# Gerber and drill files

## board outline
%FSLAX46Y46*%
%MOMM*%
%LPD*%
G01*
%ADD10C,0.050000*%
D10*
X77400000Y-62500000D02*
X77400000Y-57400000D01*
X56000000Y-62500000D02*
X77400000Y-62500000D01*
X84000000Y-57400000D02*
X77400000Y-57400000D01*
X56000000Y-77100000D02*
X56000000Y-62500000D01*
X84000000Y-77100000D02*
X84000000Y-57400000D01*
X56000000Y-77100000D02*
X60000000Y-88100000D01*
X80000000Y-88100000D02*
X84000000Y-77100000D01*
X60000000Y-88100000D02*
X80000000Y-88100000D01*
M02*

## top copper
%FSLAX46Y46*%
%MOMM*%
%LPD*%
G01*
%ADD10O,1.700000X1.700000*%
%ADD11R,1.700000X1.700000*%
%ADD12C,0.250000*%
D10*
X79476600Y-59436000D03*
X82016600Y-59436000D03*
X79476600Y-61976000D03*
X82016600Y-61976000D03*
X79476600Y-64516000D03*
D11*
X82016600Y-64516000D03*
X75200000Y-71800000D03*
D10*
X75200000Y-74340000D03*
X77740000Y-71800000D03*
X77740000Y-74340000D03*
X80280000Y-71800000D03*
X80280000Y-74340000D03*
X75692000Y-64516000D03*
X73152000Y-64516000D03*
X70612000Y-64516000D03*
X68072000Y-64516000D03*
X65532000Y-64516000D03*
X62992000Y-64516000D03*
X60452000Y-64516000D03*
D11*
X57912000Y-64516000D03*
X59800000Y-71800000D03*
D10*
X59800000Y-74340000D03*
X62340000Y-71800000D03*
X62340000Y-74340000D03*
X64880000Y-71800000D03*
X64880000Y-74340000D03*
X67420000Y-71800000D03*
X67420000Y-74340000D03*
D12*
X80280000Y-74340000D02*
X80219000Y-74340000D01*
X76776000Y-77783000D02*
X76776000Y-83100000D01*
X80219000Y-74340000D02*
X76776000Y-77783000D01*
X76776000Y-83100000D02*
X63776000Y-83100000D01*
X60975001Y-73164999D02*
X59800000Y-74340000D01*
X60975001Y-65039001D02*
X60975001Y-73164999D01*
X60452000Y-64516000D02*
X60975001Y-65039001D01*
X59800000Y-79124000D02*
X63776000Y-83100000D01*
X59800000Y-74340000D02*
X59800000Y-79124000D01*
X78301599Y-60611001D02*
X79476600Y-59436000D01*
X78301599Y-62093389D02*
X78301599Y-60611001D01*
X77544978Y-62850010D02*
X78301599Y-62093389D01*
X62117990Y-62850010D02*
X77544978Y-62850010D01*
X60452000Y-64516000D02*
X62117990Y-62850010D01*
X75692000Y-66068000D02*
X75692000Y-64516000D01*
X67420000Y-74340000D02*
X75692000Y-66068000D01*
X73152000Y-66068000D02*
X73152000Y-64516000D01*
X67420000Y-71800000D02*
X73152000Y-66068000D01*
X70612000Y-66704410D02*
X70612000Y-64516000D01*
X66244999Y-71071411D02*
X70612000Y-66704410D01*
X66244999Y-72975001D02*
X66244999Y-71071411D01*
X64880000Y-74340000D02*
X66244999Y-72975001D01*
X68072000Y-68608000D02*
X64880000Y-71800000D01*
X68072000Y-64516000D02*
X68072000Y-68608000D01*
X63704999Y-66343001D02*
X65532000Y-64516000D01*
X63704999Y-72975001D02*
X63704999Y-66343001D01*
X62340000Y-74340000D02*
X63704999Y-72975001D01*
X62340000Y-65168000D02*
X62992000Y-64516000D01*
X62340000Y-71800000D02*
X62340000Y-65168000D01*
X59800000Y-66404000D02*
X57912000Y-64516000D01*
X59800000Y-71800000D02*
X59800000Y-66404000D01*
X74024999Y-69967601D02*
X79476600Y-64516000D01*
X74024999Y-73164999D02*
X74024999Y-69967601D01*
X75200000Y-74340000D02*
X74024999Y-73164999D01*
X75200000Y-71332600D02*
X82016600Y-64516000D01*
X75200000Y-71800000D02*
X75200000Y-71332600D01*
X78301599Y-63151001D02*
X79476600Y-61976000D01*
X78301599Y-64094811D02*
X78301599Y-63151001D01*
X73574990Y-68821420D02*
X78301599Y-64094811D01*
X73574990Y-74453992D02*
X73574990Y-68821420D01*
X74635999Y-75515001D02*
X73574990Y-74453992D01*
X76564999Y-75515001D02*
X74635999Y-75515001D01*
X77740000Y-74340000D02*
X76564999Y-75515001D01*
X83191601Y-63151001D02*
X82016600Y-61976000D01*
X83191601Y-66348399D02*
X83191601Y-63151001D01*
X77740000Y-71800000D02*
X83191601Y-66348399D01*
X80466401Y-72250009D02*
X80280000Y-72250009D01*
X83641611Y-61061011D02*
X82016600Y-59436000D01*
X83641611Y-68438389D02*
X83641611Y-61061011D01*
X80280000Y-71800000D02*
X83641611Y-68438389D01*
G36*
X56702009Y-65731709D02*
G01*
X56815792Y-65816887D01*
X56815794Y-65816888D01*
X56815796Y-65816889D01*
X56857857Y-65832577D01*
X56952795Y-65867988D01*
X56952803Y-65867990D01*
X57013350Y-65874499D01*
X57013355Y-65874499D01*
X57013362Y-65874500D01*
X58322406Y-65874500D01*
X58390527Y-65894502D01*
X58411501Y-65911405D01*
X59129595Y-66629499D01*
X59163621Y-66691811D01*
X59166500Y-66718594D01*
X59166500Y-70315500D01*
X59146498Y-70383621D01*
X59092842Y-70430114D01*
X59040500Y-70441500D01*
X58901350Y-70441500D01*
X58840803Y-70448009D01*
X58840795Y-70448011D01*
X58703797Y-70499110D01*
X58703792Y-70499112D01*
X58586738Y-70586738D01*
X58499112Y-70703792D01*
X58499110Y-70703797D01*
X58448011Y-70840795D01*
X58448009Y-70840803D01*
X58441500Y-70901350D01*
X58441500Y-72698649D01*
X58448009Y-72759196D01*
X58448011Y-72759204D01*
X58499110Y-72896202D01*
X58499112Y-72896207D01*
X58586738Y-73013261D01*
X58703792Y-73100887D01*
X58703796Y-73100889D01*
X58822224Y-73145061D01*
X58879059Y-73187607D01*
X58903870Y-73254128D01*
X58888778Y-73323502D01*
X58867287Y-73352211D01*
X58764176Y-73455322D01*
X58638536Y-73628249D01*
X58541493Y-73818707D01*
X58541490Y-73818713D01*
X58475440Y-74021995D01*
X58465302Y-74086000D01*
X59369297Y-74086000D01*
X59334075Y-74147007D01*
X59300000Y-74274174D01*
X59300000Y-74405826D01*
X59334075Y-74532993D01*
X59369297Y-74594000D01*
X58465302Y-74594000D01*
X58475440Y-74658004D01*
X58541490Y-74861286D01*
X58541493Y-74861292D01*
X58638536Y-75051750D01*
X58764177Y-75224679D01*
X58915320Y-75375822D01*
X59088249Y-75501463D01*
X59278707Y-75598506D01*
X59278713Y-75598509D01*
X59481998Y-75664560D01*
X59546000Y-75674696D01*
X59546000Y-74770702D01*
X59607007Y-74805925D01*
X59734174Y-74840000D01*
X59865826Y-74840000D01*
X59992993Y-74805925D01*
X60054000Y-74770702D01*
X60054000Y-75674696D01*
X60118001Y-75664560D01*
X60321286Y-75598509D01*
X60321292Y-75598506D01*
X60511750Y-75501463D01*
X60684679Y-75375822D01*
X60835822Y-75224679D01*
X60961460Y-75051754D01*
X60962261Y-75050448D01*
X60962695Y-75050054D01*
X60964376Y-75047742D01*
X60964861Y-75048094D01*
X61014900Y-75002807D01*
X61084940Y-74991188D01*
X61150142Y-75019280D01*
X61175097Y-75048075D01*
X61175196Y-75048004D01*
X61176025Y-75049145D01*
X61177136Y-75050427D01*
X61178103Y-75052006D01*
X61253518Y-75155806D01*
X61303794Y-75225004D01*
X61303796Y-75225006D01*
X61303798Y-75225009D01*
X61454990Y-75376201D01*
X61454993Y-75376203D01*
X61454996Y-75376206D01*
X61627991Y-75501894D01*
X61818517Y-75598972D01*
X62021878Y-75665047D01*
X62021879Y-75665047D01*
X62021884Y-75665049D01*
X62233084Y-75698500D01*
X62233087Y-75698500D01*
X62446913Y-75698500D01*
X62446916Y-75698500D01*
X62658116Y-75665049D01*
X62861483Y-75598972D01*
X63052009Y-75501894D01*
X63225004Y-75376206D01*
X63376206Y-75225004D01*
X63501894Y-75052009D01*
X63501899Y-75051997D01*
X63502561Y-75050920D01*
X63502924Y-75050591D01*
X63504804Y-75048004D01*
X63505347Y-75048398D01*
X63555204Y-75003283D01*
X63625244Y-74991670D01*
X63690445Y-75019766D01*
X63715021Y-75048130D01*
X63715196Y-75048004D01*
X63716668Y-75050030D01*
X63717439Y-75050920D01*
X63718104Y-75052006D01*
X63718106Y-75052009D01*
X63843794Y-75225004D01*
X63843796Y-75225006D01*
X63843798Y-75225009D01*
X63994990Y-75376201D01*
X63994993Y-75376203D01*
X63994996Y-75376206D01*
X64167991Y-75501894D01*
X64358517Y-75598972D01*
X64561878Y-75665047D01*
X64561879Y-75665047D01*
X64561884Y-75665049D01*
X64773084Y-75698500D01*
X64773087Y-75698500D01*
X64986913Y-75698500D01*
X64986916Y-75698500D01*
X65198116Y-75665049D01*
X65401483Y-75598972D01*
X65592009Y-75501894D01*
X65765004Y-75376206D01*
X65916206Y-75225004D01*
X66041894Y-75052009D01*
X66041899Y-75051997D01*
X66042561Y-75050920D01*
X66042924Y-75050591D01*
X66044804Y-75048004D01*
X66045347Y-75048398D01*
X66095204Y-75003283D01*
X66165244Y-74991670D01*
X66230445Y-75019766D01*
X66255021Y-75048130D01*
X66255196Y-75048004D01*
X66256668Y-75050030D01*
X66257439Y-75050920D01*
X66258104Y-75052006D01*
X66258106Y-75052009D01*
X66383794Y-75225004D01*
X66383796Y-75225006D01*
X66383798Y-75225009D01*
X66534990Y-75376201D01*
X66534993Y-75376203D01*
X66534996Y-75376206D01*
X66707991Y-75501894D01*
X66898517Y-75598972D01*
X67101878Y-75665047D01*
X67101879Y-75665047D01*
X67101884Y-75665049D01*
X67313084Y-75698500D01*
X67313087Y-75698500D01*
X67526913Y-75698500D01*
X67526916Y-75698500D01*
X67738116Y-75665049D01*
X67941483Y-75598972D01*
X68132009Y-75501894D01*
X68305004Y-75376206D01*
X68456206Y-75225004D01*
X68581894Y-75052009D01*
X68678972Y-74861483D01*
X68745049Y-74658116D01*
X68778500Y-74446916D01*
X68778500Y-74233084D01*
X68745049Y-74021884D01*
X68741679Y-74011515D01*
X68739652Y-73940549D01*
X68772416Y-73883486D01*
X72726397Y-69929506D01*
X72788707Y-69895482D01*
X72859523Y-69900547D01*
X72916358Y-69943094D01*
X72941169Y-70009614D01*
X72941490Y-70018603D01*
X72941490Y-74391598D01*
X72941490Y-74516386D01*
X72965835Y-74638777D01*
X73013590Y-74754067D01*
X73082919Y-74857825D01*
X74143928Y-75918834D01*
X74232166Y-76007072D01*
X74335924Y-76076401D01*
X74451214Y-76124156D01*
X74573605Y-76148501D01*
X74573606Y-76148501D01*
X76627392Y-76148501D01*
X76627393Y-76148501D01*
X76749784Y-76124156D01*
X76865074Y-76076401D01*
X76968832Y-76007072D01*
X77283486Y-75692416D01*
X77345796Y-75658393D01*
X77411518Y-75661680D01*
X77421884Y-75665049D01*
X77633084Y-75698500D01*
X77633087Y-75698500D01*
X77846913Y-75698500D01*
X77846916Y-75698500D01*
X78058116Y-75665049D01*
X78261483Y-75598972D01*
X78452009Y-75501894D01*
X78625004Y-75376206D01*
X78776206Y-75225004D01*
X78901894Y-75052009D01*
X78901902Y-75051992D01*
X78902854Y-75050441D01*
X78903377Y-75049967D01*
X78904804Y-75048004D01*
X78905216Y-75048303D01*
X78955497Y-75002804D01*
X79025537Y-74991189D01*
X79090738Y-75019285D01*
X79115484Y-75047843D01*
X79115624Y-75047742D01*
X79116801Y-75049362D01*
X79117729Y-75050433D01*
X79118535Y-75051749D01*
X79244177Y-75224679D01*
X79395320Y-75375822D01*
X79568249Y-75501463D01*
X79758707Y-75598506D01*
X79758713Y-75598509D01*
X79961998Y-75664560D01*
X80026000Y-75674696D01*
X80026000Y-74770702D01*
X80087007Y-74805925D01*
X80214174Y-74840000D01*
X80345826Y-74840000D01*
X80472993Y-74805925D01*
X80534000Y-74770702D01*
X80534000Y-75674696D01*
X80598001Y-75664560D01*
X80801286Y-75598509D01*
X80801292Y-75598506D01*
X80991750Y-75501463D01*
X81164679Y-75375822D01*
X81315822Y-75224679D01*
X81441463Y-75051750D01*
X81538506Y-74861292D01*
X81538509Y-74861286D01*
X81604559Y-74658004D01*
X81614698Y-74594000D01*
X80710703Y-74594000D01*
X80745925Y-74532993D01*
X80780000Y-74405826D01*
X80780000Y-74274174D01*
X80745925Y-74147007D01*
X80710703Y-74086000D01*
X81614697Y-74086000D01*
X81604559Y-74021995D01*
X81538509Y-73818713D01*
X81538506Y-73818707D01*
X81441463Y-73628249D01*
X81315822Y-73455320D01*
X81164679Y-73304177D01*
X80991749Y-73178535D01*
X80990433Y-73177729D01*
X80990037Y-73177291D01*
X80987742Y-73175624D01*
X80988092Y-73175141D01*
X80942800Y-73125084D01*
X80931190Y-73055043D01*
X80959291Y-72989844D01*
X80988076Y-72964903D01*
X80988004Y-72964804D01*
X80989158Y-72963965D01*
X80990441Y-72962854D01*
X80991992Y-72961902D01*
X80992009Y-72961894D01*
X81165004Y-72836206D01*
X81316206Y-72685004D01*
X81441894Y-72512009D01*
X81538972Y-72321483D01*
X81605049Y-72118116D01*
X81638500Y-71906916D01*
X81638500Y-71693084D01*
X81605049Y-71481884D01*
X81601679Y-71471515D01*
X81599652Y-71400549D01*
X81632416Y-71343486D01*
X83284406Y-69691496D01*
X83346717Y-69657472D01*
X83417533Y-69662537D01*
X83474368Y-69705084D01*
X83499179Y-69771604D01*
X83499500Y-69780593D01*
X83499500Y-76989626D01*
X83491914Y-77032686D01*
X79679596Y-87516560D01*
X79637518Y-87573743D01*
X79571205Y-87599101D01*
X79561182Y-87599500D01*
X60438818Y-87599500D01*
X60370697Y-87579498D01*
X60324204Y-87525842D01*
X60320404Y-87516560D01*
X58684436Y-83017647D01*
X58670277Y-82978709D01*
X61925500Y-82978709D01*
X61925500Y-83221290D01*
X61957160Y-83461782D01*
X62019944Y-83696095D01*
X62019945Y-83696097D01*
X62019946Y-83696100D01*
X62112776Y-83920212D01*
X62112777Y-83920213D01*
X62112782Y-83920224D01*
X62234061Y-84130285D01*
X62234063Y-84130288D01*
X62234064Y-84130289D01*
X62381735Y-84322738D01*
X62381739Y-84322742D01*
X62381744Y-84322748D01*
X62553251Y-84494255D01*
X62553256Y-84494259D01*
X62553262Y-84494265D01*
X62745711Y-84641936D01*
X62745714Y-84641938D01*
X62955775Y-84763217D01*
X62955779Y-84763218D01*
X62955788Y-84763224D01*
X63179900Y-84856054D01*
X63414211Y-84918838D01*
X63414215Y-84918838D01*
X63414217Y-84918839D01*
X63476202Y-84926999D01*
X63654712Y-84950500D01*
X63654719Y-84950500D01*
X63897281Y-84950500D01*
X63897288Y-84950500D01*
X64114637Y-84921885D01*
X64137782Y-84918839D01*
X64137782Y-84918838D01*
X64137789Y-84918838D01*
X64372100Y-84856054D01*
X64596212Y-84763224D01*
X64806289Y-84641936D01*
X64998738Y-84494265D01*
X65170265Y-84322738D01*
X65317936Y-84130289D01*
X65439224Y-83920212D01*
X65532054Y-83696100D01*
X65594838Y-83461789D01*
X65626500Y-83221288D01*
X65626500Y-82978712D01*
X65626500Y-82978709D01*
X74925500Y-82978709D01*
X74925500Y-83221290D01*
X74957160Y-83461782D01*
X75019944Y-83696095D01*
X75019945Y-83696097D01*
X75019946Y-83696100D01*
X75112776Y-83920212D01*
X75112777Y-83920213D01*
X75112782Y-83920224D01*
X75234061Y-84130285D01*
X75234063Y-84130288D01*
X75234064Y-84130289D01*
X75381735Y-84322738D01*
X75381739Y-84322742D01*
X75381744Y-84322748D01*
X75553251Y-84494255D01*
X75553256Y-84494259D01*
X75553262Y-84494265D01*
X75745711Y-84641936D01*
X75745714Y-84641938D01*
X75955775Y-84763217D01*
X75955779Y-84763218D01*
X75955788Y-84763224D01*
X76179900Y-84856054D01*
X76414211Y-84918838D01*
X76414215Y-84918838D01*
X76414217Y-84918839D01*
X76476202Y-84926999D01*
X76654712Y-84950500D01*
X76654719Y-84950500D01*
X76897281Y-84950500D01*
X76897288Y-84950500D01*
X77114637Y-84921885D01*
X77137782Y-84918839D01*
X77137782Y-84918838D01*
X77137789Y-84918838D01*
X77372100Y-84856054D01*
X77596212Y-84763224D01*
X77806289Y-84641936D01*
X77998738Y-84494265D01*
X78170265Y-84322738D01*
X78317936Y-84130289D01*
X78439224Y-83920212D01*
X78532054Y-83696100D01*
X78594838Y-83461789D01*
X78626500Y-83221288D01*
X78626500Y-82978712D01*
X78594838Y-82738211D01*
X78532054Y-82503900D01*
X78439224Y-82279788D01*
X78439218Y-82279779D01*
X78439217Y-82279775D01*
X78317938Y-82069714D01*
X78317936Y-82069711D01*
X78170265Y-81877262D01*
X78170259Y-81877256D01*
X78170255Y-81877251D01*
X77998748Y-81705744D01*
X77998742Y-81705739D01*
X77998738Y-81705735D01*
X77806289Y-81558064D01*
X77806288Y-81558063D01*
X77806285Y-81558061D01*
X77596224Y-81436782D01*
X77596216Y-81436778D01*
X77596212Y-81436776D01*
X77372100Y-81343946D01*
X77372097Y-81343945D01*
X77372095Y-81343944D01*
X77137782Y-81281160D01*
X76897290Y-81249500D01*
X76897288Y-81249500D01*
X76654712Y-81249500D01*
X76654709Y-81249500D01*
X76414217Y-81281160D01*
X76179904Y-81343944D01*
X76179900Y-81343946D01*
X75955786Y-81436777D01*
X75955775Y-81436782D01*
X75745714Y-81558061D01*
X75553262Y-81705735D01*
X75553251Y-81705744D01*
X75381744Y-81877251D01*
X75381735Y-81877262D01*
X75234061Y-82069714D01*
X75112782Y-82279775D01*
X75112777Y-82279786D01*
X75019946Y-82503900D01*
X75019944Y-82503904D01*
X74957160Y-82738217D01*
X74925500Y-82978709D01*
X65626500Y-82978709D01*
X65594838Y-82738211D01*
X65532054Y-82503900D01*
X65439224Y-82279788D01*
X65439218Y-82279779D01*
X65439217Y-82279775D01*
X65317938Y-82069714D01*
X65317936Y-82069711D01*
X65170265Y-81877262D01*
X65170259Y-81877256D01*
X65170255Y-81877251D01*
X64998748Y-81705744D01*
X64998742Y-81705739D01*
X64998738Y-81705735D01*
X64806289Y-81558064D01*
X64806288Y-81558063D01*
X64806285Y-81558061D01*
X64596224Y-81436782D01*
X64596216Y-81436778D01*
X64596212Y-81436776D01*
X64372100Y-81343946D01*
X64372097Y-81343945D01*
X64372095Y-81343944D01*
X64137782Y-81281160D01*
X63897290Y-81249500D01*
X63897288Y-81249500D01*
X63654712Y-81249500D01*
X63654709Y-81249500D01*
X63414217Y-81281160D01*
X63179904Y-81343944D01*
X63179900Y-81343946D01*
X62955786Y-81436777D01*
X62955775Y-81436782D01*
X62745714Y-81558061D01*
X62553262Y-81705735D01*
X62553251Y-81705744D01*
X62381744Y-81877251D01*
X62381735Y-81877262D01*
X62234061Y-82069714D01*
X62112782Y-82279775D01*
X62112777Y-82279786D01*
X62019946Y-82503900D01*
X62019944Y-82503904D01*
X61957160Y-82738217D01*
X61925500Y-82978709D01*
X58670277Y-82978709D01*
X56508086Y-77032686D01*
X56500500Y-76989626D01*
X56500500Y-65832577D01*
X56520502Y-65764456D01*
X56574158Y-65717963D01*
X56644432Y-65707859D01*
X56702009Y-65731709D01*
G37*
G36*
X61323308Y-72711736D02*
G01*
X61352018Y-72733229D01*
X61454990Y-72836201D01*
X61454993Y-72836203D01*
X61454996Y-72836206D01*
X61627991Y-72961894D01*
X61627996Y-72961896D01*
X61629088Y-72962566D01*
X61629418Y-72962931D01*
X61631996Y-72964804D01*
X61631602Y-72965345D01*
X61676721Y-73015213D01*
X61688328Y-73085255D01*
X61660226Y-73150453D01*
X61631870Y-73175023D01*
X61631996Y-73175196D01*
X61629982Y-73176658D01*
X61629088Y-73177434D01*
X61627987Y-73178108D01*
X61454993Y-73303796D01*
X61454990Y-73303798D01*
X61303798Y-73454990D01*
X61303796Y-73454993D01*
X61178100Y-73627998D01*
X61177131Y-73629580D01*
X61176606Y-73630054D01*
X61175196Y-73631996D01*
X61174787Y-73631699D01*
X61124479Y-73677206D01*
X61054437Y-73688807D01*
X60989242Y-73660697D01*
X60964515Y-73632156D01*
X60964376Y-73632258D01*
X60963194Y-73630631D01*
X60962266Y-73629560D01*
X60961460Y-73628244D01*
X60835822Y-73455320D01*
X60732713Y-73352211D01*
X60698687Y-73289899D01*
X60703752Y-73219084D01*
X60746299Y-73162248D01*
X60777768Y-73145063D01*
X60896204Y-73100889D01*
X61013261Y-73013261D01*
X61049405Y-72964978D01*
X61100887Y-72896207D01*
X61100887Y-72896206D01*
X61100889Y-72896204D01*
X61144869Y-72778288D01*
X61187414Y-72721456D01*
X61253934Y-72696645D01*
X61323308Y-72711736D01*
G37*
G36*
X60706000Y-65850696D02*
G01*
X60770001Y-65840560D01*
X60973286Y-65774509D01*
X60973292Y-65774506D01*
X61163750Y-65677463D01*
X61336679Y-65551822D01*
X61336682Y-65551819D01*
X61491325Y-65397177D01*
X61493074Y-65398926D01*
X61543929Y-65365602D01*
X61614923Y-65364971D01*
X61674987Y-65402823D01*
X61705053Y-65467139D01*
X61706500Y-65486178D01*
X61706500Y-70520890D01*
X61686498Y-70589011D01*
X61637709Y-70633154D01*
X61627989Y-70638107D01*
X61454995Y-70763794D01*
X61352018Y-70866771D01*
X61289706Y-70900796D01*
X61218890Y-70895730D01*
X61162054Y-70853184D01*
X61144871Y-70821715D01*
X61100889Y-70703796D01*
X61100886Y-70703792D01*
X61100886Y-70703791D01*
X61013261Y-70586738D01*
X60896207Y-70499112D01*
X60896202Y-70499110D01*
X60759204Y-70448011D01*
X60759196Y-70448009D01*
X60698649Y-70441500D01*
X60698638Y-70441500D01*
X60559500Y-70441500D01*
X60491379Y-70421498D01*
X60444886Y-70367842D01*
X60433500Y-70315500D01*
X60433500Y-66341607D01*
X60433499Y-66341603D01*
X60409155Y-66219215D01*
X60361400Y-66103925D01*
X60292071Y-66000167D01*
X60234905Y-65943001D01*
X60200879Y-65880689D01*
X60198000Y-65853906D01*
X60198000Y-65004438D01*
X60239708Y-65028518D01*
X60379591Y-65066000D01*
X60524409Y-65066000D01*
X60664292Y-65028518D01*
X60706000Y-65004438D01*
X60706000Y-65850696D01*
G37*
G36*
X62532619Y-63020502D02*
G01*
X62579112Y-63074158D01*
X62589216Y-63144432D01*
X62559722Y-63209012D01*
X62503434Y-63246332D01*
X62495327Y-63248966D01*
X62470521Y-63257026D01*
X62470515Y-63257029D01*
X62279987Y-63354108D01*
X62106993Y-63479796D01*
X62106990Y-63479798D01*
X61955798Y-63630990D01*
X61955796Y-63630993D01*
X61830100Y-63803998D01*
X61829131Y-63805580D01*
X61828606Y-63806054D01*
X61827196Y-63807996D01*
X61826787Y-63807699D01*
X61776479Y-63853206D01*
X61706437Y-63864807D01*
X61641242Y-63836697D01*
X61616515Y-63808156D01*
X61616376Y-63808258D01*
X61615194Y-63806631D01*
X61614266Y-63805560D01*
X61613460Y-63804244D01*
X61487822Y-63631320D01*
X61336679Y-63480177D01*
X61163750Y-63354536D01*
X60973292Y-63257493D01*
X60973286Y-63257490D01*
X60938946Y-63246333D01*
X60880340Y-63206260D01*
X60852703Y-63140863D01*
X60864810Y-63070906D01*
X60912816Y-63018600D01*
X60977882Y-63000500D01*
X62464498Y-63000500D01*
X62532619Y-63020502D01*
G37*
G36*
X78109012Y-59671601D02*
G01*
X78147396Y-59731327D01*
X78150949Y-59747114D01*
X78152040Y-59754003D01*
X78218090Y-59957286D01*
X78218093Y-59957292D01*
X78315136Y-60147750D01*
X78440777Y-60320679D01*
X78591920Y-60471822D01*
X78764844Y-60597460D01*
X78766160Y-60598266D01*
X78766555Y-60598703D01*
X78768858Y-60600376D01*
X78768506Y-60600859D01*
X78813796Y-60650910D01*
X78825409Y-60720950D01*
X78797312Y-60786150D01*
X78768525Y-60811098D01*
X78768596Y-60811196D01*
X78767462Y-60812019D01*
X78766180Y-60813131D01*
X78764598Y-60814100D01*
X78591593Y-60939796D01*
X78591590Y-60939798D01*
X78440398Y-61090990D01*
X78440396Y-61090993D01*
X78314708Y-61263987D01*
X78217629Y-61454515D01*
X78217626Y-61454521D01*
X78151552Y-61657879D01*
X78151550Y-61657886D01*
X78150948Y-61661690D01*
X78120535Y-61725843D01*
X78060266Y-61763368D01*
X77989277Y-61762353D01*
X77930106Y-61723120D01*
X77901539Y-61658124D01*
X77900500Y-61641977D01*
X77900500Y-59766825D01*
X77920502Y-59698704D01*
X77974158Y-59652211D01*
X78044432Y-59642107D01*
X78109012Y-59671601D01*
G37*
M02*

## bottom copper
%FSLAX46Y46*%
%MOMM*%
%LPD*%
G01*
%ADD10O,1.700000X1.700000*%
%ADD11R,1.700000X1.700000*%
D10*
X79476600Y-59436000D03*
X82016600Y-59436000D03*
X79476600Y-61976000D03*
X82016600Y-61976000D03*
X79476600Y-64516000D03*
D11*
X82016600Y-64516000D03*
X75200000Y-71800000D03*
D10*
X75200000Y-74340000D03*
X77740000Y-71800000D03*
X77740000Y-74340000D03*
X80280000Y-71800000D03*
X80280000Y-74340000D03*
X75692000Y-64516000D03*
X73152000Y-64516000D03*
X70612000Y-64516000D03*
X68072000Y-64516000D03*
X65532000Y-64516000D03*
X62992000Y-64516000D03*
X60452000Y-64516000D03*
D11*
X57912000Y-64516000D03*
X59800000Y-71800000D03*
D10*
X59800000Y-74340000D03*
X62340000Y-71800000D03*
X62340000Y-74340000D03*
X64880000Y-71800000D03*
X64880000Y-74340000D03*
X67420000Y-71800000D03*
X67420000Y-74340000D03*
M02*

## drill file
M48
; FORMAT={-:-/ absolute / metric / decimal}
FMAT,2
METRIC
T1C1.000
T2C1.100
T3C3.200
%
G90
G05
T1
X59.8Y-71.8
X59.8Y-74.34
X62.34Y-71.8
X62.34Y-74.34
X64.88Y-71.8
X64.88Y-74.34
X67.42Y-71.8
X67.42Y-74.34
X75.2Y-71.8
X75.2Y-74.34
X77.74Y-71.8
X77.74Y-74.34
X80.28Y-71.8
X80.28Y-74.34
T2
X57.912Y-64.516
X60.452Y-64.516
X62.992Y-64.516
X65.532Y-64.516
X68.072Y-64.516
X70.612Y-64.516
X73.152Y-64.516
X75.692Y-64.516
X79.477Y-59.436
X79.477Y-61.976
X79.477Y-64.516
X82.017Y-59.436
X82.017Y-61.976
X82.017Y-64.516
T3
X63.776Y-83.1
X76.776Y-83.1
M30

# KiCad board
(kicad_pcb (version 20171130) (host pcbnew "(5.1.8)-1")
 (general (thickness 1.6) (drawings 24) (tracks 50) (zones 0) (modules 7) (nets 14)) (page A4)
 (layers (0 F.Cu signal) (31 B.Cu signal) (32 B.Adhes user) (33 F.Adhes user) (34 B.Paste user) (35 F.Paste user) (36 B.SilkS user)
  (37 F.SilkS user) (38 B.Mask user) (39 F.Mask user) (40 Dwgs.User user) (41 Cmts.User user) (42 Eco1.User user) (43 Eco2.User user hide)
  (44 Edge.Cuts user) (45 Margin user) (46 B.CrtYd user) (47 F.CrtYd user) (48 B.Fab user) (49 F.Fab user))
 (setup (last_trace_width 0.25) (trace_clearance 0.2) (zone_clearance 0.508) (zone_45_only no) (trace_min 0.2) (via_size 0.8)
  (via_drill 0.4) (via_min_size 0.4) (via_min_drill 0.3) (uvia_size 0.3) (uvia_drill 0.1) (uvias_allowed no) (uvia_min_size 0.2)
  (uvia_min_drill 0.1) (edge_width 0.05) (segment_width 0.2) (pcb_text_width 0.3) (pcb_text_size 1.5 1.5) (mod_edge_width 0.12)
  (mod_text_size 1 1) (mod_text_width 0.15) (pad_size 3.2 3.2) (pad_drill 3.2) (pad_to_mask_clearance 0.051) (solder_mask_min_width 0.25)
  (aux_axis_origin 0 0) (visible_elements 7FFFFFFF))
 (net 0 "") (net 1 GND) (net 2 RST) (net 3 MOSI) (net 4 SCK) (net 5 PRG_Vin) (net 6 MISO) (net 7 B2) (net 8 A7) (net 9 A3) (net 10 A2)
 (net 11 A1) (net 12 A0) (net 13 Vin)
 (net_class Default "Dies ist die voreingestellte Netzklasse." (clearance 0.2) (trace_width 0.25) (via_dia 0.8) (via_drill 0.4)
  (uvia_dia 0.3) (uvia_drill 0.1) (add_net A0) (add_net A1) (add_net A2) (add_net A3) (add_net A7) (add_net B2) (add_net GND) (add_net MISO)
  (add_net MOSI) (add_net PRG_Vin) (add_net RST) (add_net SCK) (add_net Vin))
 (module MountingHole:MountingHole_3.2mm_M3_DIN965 (layer F.Cu) (at 63.6778 83.1342)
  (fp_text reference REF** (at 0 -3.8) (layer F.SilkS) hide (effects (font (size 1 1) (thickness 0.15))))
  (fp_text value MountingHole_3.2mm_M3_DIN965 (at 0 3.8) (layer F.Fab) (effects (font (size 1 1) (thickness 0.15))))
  (pad "" np_thru_hole circle (at 0.0982 -0.0342) (size 3.2 3.2) (drill 3.2) (layers *.Cu *.Mask)))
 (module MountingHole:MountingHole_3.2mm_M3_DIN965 (layer F.Cu) (at 76.776 83.1)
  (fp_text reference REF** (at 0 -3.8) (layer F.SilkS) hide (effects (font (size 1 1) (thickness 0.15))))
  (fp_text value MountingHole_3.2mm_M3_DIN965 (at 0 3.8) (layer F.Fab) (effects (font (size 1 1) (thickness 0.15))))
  (pad 1 np_thru_hole circle (at 0 0) (size 3.2 3.2) (drill 3.2) (layers *.Cu *.Mask)))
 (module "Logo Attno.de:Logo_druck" (layer F.Cu) (at 70.2056 82.042)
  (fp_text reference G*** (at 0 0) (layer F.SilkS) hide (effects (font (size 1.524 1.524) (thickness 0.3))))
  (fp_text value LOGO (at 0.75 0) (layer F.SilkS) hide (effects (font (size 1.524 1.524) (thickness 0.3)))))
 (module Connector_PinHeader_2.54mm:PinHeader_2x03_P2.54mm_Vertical (layer F.Cu) (at 82.0166 64.516 180)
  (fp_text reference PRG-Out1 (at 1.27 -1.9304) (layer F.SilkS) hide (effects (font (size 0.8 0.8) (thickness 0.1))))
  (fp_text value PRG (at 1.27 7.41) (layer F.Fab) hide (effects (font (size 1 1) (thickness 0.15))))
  (pad 6 thru_hole oval (at 2.54 5.08 180) (size 1.7 1.7) (drill 1.1) (layers *.Cu *.Mask) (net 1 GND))
  (pad 5 thru_hole oval (at 0 5.08 180) (size 1.7 1.7) (drill 1.1) (layers *.Cu *.Mask) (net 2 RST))
  (pad 4 thru_hole oval (at 2.54 2.54 180) (size 1.7 1.7) (drill 1.1) (layers *.Cu *.Mask) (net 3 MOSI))
  (pad 3 thru_hole oval (at 0 2.54 180) (size 1.7 1.7) (drill 1.1) (layers *.Cu *.Mask) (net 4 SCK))
  (pad 2 thru_hole oval (at 2.54 0 180) (size 1.7 1.7) (drill 1.1) (layers *.Cu *.Mask) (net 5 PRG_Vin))
  (pad 1 thru_hole rect (at 0 0 180) (size 1.7 1.7) (drill 1.1) (layers *.Cu *.Mask) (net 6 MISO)))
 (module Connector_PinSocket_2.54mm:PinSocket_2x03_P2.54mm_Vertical (layer F.Cu) (at 75.2 71.8 90)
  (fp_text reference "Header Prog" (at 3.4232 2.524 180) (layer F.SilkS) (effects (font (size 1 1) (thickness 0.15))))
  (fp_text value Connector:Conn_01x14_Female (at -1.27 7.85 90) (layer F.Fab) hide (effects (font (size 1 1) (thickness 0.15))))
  (pad 1 thru_hole rect (at 0 0 90) (size 1.7 1.7) (drill 1) (layers *.Cu *.Mask) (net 6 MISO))
  (pad 2 thru_hole oval (at -2.54 0 90) (size 1.7 1.7) (drill 1) (layers *.Cu *.Mask) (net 5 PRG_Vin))
  (pad 3 thru_hole oval (at 0 2.54 90) (size 1.7 1.7) (drill 1) (layers *.Cu *.Mask) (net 4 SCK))
  (pad 4 thru_hole oval (at -2.54 2.54 90) (size 1.7 1.7) (drill 1) (layers *.Cu *.Mask) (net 3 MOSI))
  (pad 5 thru_hole oval (at 0 5.08 90) (size 1.7 1.7) (drill 1) (layers *.Cu *.Mask) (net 2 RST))
  (pad 6 thru_hole oval (at -2.54 5.08 90) (size 1.7 1.7) (drill 1) (layers *.Cu *.Mask) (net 1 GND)))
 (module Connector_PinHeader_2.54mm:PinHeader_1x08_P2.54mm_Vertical (layer F.Cu) (at 57.912 64.516 90)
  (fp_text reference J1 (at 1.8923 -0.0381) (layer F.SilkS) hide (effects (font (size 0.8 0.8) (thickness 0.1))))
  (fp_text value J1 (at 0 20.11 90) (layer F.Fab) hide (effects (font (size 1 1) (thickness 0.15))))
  (pad 8 thru_hole oval (at 0 17.78 90) (size 1.7 1.7) (drill 1.1) (layers *.Cu *.Mask) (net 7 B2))
  (pad 7 thru_hole oval (at 0 15.24 90) (size 1.7 1.7) (drill 1.1) (layers *.Cu *.Mask) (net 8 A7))
  (pad 6 thru_hole oval (at 0 12.7 90) (size 1.7 1.7) (drill 1.1) (layers *.Cu *.Mask) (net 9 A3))
  (pad 5 thru_hole oval (at 0 10.16 90) (size 1.7 1.7) (drill 1.1) (layers *.Cu *.Mask) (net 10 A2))
  (pad 4 thru_hole oval (at 0 7.62 90) (size 1.7 1.7) (drill 1.1) (layers *.Cu *.Mask) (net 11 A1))
  (pad 3 thru_hole oval (at 0 5.08 90) (size 1.7 1.7) (drill 1.1) (layers *.Cu *.Mask) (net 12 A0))
  (pad 2 thru_hole oval (at 0 2.54 90) (size 1.7 1.7) (drill 1.1) (layers *.Cu *.Mask) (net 1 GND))
  (pad 1 thru_hole rect (at 0 0 90) (size 1.7 1.7) (drill 1.1) (layers *.Cu *.Mask) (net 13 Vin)))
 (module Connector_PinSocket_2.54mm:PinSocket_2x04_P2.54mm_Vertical (layer F.Cu) (at 59.8 71.8 90)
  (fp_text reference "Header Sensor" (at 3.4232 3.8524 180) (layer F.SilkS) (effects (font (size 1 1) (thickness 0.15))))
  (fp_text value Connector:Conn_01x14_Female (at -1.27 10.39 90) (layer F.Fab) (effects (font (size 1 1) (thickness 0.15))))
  (pad 1 thru_hole rect (at 0 0 90) (size 1.7 1.7) (drill 1) (layers *.Cu *.Mask) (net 13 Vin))
  (pad 2 thru_hole oval (at -2.54 0 90) (size 1.7 1.7) (drill 1) (layers *.Cu *.Mask) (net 1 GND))
  (pad 3 thru_hole oval (at 0 2.54 90) (size 1.7 1.7) (drill 1) (layers *.Cu *.Mask) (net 12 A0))
  (pad 4 thru_hole oval (at -2.54 2.54 90) (size 1.7 1.7) (drill 1) (layers *.Cu *.Mask) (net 11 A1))
  (pad 5 thru_hole oval (at 0 5.08 90) (size 1.7 1.7) (drill 1) (layers *.Cu *.Mask) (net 10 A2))
  (pad 6 thru_hole oval (at -2.54 5.08 90) (size 1.7 1.7) (drill 1) (layers *.Cu *.Mask) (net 9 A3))
  (pad 7 thru_hole oval (at 0 7.62 90) (size 1.7 1.7) (drill 1) (layers *.Cu *.Mask) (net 8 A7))
  (pad 8 thru_hole oval (at -2.54 7.62 90) (size 1.7 1.7) (drill 1) (layers *.Cu *.Mask) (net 7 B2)))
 (gr_line (start 77.4 62.5) (end 77.4 57.4) (layer Edge.Cuts) (width 0.05))
 (gr_line (start 56 62.5) (end 77.4 62.5) (layer Edge.Cuts) (width 0.05))
 (gr_line (start 84 57.4) (end 77.4 57.4) (layer Edge.Cuts) (width 0.05))
 (gr_line (start 56 77.1) (end 56 62.5) (layer Edge.Cuts) (width 0.05))
 (gr_line (start 84 77.1) (end 84 57.4) (layer Edge.Cuts) (width 0.05))
 (gr_line (start 56 77.1) (end 60 88.1) (layer Edge.Cuts) (width 0.05))
 (gr_line (start 80 88.1) (end 84 77.1) (layer Edge.Cuts) (width 0.05))
 (gr_line (start 60 88.1) (end 80 88.1) (layer Edge.Cuts) (width 0.05))
 (segment (start 80.28 74.34) (end 80.219 74.34) (width 0.25) (layer F.Cu) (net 1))
 (segment (start 76.776 77.783) (end 76.776 83.1) (width 0.25) (layer F.Cu) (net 1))
 (segment (start 80.219 74.34) (end 76.776 77.783) (width 0.25) (layer F.Cu) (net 1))
 (segment (start 76.776 83.1) (end 63.776 83.1) (width 0.25) (layer F.Cu) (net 1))
 (segment (start 60.975001 73.164999) (end 59.8 74.34) (width 0.25) (layer F.Cu) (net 1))
 (segment (start 60.975001 65.039001) (end 60.975001 73.164999) (width 0.25) (layer F.Cu) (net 1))
 (segment (start 60.452 64.516) (end 60.975001 65.039001) (width 0.25) (layer F.Cu) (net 1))
 (segment (start 59.8 79.124) (end 63.776 83.1) (width 0.25) (layer F.Cu) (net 1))
 (segment (start 59.8 74.34) (end 59.8 79.124) (width 0.25) (layer F.Cu) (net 1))
 (segment (start 78.301599 60.611001) (end 79.4766 59.436) (width 0.25) (layer F.Cu) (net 1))
 (segment (start 78.301599 62.093389) (end 78.301599 60.611001) (width 0.25) (layer F.Cu) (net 1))
 (segment (start 77.544978 62.85001) (end 78.301599 62.093389) (width 0.25) (layer F.Cu) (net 1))
 (segment (start 62.11799 62.85001) (end 77.544978 62.85001) (width 0.25) (layer F.Cu) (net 1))
 (segment (start 60.452 64.516) (end 62.11799 62.85001) (width 0.25) (layer F.Cu) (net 1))
 (segment (start 75.692 66.068) (end 75.692 64.516) (width 0.25) (layer F.Cu) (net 7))
 (segment (start 67.42 74.34) (end 75.692 66.068) (width 0.25) (layer F.Cu) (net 7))
 (segment (start 73.152 66.068) (end 73.152 64.516) (width 0.25) (layer F.Cu) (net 8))
 (segment (start 67.42 71.8) (end 73.152 66.068) (width 0.25) (layer F.Cu) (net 8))
 (segment (start 70.612 66.70441) (end 70.612 64.516) (width 0.25) (layer F.Cu) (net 9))
 (segment (start 66.244999 71.071411) (end 70.612 66.70441) (width 0.25) (layer F.Cu) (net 9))
 (segment (start 66.244999 72.975001) (end 66.244999 71.071411) (width 0.25) (layer F.Cu) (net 9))
 (segment (start 64.88 74.34) (end 66.244999 72.975001) (width 0.25) (layer F.Cu) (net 9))
 (segment (start 68.072 68.608) (end 64.88 71.8) (width 0.25) (layer F.Cu) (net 10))
 (segment (start 68.072 64.516) (end 68.072 68.608) (width 0.25) (layer F.Cu) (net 10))
 (segment (start 63.704999 66.343001) (end 65.532 64.516) (width 0.25) (layer F.Cu) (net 11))
 (segment (start 63.704999 72.975001) (end 63.704999 66.343001) (width 0.25) (layer F.Cu) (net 11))
 (segment (start 62.34 74.34) (end 63.704999 72.975001) (width 0.25) (layer F.Cu) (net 11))
 (segment (start 62.34 65.168) (end 62.992 64.516) (width 0.25) (layer F.Cu) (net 12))
 (segment (start 62.34 71.8) (end 62.34 65.168) (width 0.25) (layer F.Cu) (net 12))
 (segment (start 59.8 66.404) (end 57.912 64.516) (width 0.25) (layer F.Cu) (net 13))
 (segment (start 59.8 71.8) (end 59.8 66.404) (width 0.25) (layer F.Cu) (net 13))
 (segment (start 74.024999 69.967601) (end 79.4766 64.516) (width 0.25) (layer F.Cu) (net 5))
 (segment (start 74.024999 73.164999) (end 74.024999 69.967601) (width 0.25) (layer F.Cu) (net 5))
 (segment (start 75.2 74.34) (end 74.024999 73.164999) (width 0.25) (layer F.Cu) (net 5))
 (segment (start 75.2 71.3326) (end 82.0166 64.516) (width 0.25) (layer F.Cu) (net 6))
 (segment (start 75.2 71.8) (end 75.2 71.3326) (width 0.25) (layer F.Cu) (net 6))
 (segment (start 78.301599 63.151001) (end 79.4766 61.976) (width 0.25) (layer F.Cu) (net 3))
 (segment (start 78.301599 64.094811) (end 78.301599 63.151001) (width 0.25) (layer F.Cu) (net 3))
 (segment (start 73.57499 68.82142) (end 78.301599 64.094811) (width 0.25) (layer F.Cu) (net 3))
 (segment (start 73.57499 74.453992) (end 73.57499 68.82142) (width 0.25) (layer F.Cu) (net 3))
 (segment (start 74.635999 75.515001) (end 73.57499 74.453992) (width 0.25) (layer F.Cu) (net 3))
 (segment (start 76.564999 75.515001) (end 74.635999 75.515001) (width 0.25) (layer F.Cu) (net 3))
 (segment (start 77.74 74.34) (end 76.564999 75.515001) (width 0.25) (layer F.Cu) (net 3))
 (segment (start 83.191601 63.151001) (end 82.0166 61.976) (width 0.25) (layer F.Cu) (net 4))
 (segment (start 83.191601 66.348399) (end 83.191601 63.151001) (width 0.25) (layer F.Cu) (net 4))
 (segment (start 77.74 71.8) (end 83.191601 66.348399) (width 0.25) (layer F.Cu) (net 4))
 (segment (start 80.466401 72.250009) (end 80.28 72.250009) (width 0.25) (layer F.Cu) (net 2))
 (segment (start 83.641611 61.061011) (end 82.0166 59.436) (width 0.25) (layer F.Cu) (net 2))
 (segment (start 83.641611 68.438389) (end 83.641611 61.061011) (width 0.25) (layer F.Cu) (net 2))
 (segment (start 80.28 71.8) (end 83.641611 68.438389) (width 0.25) (layer F.Cu) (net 2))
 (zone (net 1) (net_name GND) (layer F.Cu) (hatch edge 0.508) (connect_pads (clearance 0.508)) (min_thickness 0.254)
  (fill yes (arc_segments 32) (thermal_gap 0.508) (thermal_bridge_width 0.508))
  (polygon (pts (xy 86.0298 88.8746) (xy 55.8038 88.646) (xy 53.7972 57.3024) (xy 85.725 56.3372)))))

